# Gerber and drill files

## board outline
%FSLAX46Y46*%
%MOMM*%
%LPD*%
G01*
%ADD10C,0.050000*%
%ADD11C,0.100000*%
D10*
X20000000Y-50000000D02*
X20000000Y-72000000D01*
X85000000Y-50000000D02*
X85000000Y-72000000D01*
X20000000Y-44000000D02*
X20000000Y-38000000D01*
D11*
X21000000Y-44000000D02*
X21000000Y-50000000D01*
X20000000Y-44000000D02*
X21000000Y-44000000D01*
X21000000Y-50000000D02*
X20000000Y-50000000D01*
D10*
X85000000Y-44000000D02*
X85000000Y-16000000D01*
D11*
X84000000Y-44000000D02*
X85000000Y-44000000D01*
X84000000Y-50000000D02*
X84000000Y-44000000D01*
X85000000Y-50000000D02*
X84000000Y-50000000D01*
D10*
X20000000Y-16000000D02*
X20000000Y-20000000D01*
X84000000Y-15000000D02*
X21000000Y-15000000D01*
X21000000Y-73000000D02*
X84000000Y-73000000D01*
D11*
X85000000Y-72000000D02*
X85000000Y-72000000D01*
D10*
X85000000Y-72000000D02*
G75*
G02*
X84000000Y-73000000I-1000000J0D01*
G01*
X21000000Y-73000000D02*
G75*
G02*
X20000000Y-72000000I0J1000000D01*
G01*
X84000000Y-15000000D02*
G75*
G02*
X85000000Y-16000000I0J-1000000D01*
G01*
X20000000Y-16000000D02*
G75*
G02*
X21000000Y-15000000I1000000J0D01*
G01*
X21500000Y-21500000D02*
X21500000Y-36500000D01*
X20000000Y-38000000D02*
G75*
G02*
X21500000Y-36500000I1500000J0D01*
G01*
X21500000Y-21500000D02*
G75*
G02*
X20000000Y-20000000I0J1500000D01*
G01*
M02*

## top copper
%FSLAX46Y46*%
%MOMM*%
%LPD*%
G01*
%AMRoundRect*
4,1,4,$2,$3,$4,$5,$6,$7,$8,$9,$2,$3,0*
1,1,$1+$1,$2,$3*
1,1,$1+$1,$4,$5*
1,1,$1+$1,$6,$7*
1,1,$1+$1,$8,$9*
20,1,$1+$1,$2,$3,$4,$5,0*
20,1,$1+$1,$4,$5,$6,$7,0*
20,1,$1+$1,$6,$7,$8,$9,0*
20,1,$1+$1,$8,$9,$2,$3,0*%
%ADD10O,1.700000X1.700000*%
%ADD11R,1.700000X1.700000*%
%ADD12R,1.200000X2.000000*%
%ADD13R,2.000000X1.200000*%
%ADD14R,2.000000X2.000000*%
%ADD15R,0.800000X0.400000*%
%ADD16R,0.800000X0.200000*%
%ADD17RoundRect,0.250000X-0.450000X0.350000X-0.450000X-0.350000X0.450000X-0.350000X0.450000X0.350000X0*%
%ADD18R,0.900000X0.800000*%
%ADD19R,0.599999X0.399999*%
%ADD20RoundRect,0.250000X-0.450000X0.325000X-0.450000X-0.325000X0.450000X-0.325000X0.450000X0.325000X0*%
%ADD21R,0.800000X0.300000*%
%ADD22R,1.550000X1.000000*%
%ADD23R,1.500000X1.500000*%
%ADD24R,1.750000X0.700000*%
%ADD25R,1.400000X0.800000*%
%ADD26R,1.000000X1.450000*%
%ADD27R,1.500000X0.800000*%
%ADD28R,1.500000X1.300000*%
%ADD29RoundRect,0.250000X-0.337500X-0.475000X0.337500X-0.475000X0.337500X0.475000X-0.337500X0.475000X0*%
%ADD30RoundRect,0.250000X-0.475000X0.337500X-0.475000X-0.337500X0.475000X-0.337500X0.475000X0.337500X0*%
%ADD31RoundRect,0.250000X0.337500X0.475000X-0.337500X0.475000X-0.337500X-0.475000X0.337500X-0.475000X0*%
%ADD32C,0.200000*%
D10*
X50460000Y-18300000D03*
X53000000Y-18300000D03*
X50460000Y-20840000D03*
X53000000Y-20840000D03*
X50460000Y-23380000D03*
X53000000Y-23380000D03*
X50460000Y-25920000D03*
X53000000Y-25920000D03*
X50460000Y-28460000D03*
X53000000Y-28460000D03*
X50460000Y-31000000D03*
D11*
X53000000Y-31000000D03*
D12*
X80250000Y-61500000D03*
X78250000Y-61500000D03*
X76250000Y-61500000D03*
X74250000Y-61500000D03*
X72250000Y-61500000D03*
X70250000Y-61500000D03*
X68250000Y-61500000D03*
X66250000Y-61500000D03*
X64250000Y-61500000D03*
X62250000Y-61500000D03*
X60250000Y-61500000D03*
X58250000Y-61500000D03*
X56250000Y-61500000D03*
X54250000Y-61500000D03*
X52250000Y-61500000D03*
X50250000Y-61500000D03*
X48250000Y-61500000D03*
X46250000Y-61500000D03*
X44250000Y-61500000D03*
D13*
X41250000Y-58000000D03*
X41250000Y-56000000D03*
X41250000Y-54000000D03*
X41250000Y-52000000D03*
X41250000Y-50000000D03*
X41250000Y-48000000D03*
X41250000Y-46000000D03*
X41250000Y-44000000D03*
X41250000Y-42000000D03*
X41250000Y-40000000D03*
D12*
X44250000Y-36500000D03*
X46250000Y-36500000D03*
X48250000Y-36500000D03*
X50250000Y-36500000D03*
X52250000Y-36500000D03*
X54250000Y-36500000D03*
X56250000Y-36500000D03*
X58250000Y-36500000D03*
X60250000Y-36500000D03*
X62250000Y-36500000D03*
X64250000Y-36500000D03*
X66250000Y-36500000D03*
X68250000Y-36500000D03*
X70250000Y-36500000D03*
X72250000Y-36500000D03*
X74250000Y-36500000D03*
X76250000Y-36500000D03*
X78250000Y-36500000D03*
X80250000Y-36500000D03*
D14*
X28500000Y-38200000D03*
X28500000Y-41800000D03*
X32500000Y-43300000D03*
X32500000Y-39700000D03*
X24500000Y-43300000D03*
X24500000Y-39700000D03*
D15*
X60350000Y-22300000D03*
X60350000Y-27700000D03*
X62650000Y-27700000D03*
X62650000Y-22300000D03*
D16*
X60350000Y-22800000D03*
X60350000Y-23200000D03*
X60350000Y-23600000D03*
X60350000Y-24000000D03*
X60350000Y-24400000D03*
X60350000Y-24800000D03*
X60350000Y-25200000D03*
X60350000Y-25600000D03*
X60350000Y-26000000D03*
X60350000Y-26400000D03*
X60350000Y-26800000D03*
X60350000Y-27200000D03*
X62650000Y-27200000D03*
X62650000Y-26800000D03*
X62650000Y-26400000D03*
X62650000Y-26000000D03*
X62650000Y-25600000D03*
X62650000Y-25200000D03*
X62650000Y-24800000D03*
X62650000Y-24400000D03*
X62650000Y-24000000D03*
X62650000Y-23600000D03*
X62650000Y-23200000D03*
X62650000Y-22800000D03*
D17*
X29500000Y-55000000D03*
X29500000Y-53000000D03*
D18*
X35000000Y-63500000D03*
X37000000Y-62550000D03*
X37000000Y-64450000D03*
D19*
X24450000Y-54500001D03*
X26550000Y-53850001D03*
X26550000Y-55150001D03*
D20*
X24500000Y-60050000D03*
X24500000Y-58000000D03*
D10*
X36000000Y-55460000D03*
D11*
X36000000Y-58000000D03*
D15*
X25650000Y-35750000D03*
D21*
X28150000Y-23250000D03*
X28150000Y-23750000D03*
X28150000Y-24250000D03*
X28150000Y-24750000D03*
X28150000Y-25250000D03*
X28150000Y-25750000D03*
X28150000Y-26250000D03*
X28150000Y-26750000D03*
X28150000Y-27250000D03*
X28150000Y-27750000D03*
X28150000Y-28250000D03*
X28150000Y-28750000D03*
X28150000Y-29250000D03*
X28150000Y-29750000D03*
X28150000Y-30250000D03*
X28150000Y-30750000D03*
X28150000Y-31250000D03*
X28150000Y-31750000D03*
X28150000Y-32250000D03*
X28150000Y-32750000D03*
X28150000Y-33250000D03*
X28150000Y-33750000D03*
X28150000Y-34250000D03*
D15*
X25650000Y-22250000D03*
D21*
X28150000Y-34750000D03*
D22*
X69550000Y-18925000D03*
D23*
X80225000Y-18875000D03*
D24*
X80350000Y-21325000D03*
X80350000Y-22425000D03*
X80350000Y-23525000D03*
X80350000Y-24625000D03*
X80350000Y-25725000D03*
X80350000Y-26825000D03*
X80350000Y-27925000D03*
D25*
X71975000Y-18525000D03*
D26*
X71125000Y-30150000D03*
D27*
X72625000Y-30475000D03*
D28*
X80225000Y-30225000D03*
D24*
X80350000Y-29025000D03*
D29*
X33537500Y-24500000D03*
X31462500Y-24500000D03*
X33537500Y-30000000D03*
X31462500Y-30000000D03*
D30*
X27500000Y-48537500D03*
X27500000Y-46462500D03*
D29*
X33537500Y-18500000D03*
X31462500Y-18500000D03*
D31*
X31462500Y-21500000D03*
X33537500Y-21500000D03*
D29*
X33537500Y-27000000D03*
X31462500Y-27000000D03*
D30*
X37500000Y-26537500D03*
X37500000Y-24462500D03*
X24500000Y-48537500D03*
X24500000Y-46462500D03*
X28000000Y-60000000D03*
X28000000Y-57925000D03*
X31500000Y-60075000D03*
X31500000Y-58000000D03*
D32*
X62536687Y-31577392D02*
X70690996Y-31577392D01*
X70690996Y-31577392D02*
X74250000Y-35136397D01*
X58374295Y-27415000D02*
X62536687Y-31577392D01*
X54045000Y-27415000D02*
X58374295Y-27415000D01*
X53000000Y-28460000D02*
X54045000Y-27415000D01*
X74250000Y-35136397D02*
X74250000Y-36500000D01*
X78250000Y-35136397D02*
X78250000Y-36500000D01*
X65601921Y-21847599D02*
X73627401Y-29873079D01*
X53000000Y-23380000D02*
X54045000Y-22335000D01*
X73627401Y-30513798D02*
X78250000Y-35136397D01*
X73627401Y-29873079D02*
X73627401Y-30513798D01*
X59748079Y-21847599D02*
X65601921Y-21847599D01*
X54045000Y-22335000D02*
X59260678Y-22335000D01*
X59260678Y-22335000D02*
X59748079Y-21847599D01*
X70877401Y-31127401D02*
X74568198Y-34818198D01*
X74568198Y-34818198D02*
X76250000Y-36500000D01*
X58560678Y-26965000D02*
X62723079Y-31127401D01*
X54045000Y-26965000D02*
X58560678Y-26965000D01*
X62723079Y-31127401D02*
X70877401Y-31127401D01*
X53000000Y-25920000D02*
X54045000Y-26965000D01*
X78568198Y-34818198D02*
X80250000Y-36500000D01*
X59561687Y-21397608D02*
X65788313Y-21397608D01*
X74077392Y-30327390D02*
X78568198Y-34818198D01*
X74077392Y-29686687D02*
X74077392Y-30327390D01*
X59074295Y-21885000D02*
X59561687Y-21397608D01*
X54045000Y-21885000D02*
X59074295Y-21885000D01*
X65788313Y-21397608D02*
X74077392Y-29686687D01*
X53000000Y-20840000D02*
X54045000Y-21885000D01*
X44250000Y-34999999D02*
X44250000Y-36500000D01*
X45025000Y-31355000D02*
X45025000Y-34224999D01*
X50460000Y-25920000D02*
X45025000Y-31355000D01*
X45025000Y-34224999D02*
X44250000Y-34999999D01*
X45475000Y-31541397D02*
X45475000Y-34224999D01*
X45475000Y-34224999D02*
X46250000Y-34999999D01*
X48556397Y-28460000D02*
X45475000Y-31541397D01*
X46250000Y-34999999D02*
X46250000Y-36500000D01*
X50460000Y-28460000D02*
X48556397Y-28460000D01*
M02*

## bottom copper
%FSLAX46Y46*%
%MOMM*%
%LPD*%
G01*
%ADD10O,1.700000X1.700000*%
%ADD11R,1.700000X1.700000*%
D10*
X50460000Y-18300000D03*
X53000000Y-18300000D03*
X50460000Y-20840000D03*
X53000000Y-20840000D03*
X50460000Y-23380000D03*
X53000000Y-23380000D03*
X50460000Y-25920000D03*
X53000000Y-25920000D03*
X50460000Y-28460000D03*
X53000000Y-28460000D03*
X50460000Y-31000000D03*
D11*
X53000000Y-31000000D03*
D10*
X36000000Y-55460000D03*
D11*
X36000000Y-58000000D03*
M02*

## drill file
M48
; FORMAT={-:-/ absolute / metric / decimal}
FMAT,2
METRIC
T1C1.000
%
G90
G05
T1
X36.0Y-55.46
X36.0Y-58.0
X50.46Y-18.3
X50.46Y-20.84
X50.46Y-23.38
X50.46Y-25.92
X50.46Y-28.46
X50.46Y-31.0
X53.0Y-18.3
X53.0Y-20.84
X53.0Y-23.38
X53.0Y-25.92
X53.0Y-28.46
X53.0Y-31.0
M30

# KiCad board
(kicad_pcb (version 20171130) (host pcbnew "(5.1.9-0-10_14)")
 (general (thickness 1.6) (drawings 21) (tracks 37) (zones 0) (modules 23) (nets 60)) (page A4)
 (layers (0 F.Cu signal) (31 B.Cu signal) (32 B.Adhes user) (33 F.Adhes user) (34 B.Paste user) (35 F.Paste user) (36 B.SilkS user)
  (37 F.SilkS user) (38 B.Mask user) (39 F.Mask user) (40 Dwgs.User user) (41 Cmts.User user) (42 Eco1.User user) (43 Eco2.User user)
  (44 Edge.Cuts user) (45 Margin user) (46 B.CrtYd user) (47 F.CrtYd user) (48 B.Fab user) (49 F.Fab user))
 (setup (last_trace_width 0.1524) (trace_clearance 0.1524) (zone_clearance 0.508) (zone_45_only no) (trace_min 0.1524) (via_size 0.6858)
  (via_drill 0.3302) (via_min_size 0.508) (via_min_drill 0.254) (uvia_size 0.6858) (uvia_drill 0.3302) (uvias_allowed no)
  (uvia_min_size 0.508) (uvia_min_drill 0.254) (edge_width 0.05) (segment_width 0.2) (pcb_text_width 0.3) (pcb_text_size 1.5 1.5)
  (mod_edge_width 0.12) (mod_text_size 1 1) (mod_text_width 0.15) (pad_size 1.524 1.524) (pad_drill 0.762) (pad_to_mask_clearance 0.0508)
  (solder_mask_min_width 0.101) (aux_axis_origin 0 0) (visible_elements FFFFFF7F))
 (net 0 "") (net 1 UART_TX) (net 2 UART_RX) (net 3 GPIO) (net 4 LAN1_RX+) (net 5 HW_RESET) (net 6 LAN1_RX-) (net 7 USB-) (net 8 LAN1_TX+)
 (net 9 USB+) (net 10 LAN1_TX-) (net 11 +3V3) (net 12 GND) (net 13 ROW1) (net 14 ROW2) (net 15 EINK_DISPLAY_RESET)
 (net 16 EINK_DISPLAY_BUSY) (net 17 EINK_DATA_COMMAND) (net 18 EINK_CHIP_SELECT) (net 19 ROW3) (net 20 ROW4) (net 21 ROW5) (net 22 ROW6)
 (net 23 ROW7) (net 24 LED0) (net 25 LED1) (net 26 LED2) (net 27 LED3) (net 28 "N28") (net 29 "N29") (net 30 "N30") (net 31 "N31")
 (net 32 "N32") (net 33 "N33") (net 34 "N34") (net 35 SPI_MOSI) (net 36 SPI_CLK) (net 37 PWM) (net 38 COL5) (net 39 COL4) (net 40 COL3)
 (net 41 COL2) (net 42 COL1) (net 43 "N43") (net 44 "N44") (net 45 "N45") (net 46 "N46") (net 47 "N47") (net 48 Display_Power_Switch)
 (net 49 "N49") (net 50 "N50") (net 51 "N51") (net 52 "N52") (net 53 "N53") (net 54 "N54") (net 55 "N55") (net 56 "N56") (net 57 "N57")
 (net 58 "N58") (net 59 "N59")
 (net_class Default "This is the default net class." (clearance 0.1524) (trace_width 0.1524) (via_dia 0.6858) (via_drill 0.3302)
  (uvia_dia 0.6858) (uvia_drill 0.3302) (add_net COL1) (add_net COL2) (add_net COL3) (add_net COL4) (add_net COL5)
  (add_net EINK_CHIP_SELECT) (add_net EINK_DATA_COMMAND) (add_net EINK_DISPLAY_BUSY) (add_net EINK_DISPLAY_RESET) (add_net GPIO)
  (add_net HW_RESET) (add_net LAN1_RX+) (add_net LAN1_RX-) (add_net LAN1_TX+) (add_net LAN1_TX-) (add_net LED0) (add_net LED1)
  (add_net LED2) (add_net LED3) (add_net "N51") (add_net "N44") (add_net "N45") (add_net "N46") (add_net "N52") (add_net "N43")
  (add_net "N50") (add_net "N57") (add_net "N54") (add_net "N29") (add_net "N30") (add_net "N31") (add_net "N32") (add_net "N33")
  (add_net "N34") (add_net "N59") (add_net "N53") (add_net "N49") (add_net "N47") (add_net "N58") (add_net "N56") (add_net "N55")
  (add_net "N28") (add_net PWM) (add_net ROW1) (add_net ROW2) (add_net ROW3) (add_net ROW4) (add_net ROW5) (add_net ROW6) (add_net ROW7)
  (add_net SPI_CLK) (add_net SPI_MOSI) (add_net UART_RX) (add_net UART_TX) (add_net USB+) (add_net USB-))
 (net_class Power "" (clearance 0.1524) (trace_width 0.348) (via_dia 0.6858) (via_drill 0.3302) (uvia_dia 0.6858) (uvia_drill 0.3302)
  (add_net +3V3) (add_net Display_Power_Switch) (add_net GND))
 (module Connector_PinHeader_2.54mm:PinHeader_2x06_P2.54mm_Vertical (layer F.Cu) (at 53 31 180)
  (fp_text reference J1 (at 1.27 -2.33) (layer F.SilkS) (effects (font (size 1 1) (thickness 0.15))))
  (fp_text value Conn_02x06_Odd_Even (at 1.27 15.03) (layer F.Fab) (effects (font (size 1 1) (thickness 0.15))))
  (pad 12 thru_hole oval (at 2.54 12.7 180) (size 1.7 1.7) (drill 1) (layers *.Cu *.Mask) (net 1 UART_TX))
  (pad 11 thru_hole oval (at 0 12.7 180) (size 1.7 1.7) (drill 1) (layers *.Cu *.Mask) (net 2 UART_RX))
  (pad 10 thru_hole oval (at 2.54 10.16 180) (size 1.7 1.7) (drill 1) (layers *.Cu *.Mask) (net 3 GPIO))
  (pad 9 thru_hole oval (at 0 10.16 180) (size 1.7 1.7) (drill 1) (layers *.Cu *.Mask) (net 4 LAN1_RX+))
  (pad 8 thru_hole oval (at 2.54 7.62 180) (size 1.7 1.7) (drill 1) (layers *.Cu *.Mask) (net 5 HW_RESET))
  (pad 7 thru_hole oval (at 0 7.62 180) (size 1.7 1.7) (drill 1) (layers *.Cu *.Mask) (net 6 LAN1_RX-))
  (pad 6 thru_hole oval (at 2.54 5.08 180) (size 1.7 1.7) (drill 1) (layers *.Cu *.Mask) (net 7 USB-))
  (pad 5 thru_hole oval (at 0 5.08 180) (size 1.7 1.7) (drill 1) (layers *.Cu *.Mask) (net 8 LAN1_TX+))
  (pad 4 thru_hole oval (at 2.54 2.54 180) (size 1.7 1.7) (drill 1) (layers *.Cu *.Mask) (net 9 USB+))
  (pad 3 thru_hole oval (at 0 2.54 180) (size 1.7 1.7) (drill 1) (layers *.Cu *.Mask) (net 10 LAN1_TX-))
  (pad 2 thru_hole oval (at 2.54 0 180) (size 1.7 1.7) (drill 1) (layers *.Cu *.Mask) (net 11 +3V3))
  (pad 1 thru_hole rect (at 0 0 180) (size 1.7 1.7) (drill 1) (layers *.Cu *.Mask) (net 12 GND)))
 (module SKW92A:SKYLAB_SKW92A (layer F.Cu) (at 61.5 49)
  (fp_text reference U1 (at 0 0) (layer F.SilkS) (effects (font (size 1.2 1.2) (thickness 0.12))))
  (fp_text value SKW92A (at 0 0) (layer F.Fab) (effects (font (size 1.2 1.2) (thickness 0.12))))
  (pad 48 smd rect (at 18.75 12.5) (size 1.2 2) (layers F.Cu F.Paste F.Mask) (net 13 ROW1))
  (pad 47 smd rect (at 16.75 12.5) (size 1.2 2) (layers F.Cu F.Paste F.Mask) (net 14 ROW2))
  (pad 46 smd rect (at 14.75 12.5) (size 1.2 2) (layers F.Cu F.Paste F.Mask) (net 3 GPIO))
  (pad 45 smd rect (at 12.75 12.5) (size 1.2 2) (layers F.Cu F.Paste F.Mask) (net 5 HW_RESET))
  (pad 44 smd rect (at 10.75 12.5) (size 1.2 2) (layers F.Cu F.Paste F.Mask) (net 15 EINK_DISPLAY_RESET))
  (pad 43 smd rect (at 8.75 12.5) (size 1.2 2) (layers F.Cu F.Paste F.Mask) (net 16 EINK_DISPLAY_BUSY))
  (pad 42 smd rect (at 6.75 12.5) (size 1.2 2) (layers F.Cu F.Paste F.Mask) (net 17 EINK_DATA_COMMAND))
  (pad 41 smd rect (at 4.75 12.5) (size 1.2 2) (layers F.Cu F.Paste F.Mask) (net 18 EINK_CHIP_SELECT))
  (pad 40 smd rect (at 2.75 12.5) (size 1.2 2) (layers F.Cu F.Paste F.Mask) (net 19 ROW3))
  (pad 39 smd rect (at 0.75 12.5) (size 1.2 2) (layers F.Cu F.Paste F.Mask) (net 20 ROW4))
  (pad 38 smd rect (at -1.25 12.5) (size 1.2 2) (layers F.Cu F.Paste F.Mask) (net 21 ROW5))
  (pad 37 smd rect (at -3.25 12.5) (size 1.2 2) (layers F.Cu F.Paste F.Mask) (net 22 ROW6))
  (pad 36 smd rect (at -5.25 12.5) (size 1.2 2) (layers F.Cu F.Paste F.Mask) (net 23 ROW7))
  (pad 35 smd rect (at -7.25 12.5) (size 1.2 2) (layers F.Cu F.Paste F.Mask) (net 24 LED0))
  (pad 34 smd rect (at -9.25 12.5) (size 1.2 2) (layers F.Cu F.Paste F.Mask) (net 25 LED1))
  (pad 33 smd rect (at -11.25 12.5) (size 1.2 2) (layers F.Cu F.Paste F.Mask) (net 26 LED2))
  (pad 32 smd rect (at -13.25 12.5) (size 1.2 2) (layers F.Cu F.Paste F.Mask) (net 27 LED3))
  (pad 31 smd rect (at -15.25 12.5) (size 1.2 2) (layers F.Cu F.Paste F.Mask) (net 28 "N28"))
  (pad 30 smd rect (at -17.25 12.5) (size 1.2 2) (layers F.Cu F.Paste F.Mask) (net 12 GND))
  (pad 29 smd rect (at -20.25 9 90) (size 1.2 2) (layers F.Cu F.Paste F.Mask) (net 11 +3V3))
  (pad 28 smd rect (at -20.25 7 90) (size 1.2 2) (layers F.Cu F.Paste F.Mask) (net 11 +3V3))
  (pad 27 smd rect (at -20.25 5 90) (size 1.2 2) (layers F.Cu F.Paste F.Mask) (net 12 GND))
  (pad 26 smd rect (at -20.25 3 90) (size 1.2 2) (layers F.Cu F.Paste F.Mask) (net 1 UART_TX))
  (pad 25 smd rect (at -20.25 1 90) (size 1.2 2) (layers F.Cu F.Paste F.Mask) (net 2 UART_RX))
  (pad 24 smd rect (at -20.25 -1 90) (size 1.2 2) (layers F.Cu F.Paste F.Mask) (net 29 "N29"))
  (pad 23 smd rect (at -20.25 -3 90) (size 1.2 2) (layers F.Cu F.Paste F.Mask) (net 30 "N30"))
  (pad 22 smd rect (at -20.25 -5 90) (size 1.2 2) (layers F.Cu F.Paste F.Mask) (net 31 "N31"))
  (pad 21 smd rect (at -20.25 -7 90) (size 1.2 2) (layers F.Cu F.Paste F.Mask) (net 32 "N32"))
  (pad 20 smd rect (at -20.25 -9 90) (size 1.2 2) (layers F.Cu F.Paste F.Mask) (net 12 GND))
  (pad 19 smd rect (at -17.25 -12.5) (size 1.2 2) (layers F.Cu F.Paste F.Mask) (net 7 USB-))
  (pad 18 smd rect (at -15.25 -12.5) (size 1.2 2) (layers F.Cu F.Paste F.Mask) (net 9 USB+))
  (pad 17 smd rect (at -13.25 -12.5) (size 1.2 2) (layers F.Cu F.Paste F.Mask) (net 12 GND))
  (pad 16 smd rect (at -11.25 -12.5) (size 1.2 2) (layers F.Cu F.Paste F.Mask) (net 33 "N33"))
  (pad 15 smd rect (at -9.25 -12.5) (size 1.2 2) (layers F.Cu F.Paste F.Mask) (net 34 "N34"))
  (pad 14 smd rect (at -7.25 -12.5) (size 1.2 2) (layers F.Cu F.Paste F.Mask) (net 12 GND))
  (pad 13 smd rect (at -5.25 -12.5) (size 1.2 2) (layers F.Cu F.Paste F.Mask) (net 12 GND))
  (pad 12 smd rect (at -3.25 -12.5) (size 1.2 2) (layers F.Cu F.Paste F.Mask) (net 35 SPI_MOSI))
  (pad 11 smd rect (at -1.25 -12.5) (size 1.2 2) (layers F.Cu F.Paste F.Mask) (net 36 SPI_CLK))
  (pad 10 smd rect (at 0.75 -12.5) (size 1.2 2) (layers F.Cu F.Paste F.Mask) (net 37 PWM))
  (pad 9 smd rect (at 2.75 -12.5) (size 1.2 2) (layers F.Cu F.Paste F.Mask) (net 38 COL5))
  (pad 8 smd rect (at 4.75 -12.5) (size 1.2 2) (layers F.Cu F.Paste F.Mask) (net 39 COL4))
  (pad 7 smd rect (at 6.75 -12.5) (size 1.2 2) (layers F.Cu F.Paste F.Mask) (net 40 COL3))
  (pad 6 smd rect (at 8.75 -12.5) (size 1.2 2) (layers F.Cu F.Paste F.Mask) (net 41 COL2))
  (pad 5 smd rect (at 10.75 -12.5) (size 1.2 2) (layers F.Cu F.Paste F.Mask) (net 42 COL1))
  (pad 4 smd rect (at 12.75 -12.5) (size 1.2 2) (layers F.Cu F.Paste F.Mask) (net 10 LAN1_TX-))
  (pad 3 smd rect (at 14.75 -12.5) (size 1.2 2) (layers F.Cu F.Paste F.Mask) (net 8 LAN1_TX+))
  (pad 2 smd rect (at 16.75 -12.5) (size 1.2 2) (layers F.Cu F.Paste F.Mask) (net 6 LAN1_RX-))
  (pad 1 smd rect (at 18.75 -12.5) (size 1.2 2) (layers F.Cu F.Paste F.Mask) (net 4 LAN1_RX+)))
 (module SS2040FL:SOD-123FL (layer F.Cu) (at 28.5 40 90)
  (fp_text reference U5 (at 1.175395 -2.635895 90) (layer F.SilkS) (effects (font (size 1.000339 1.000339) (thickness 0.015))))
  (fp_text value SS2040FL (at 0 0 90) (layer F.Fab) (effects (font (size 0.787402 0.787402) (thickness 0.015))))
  (pad 2 smd rect (at 1.8 0 90) (size 2 2) (layers F.Cu F.Paste F.Mask) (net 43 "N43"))
  (pad 1 smd rect (at -1.8 0 90) (size 2 2) (layers F.Cu F.Paste F.Mask) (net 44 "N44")))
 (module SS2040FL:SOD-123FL (layer F.Cu) (at 32.5 41.5 270)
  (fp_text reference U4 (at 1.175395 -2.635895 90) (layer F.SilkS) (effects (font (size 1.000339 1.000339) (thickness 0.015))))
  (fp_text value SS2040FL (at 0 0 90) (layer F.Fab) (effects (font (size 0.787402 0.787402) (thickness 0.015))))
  (pad 2 smd rect (at 1.8 0 270) (size 2 2) (layers F.Cu F.Paste F.Mask) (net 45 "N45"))
  (pad 1 smd rect (at -1.8 0 270) (size 2 2) (layers F.Cu F.Paste F.Mask) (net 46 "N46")))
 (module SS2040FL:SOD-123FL (layer F.Cu) (at 24.5 41.5 270)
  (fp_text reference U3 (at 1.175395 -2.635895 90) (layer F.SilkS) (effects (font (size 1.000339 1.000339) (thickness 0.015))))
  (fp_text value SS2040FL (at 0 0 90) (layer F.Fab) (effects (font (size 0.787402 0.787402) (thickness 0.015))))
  (pad 2 smd rect (at 1.8 0 270) (size 2 2) (layers F.Cu F.Paste F.Mask) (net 44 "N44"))
  (pad 1 smd rect (at -1.8 0 270) (size 2 2) (layers F.Cu F.Paste F.Mask) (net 12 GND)))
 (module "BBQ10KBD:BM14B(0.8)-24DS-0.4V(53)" (layer F.Cu) (at 61.5 25 270)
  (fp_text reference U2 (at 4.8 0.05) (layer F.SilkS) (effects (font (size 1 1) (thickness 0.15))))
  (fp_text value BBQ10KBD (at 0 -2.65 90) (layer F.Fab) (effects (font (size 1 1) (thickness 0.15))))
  (pad 28 smd rect (at -2.7 1.15 270) (size 0.4 0.8) (layers F.Cu F.Paste F.Mask) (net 12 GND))
  (pad 15 smd rect (at 2.7 1.15 270) (size 0.4 0.8) (layers F.Cu F.Paste F.Mask) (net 12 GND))
  (pad 14 smd rect (at 2.7 -1.15 270) (size 0.4 0.8) (layers F.Cu F.Paste F.Mask) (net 12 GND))
  (pad 1 smd rect (at -2.7 -1.15 270) (size 0.4 0.8) (layers F.Cu F.Paste F.Mask) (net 12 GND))
  (pad 27 smd rect (at -2.2 1.15 270) (size 0.2 0.8) (layers F.Cu F.Paste F.Mask) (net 23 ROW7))
  (pad 26 smd rect (at -1.8 1.15 270) (size 0.2 0.8) (layers F.Cu F.Paste F.Mask) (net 24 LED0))
  (pad 25 smd rect (at -1.4 1.15 270) (size 0.2 0.8) (layers F.Cu F.Paste F.Mask) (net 26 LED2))
  (pad 24 smd rect (at -1 1.15 270) (size 0.2 0.8) (layers F.Cu F.Paste F.Mask) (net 25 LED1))
  (pad 23 smd rect (at -0.6 1.15 270) (size 0.2 0.8) (layers F.Cu F.Paste F.Mask) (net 27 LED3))
  (pad 22 smd rect (at -0.2 1.15 270) (size 0.2 0.8) (layers F.Cu F.Paste F.Mask) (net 22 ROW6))
  (pad 21 smd rect (at 0.2 1.15 270) (size 0.2 0.8) (layers F.Cu F.Paste F.Mask) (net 21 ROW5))
  (pad 20 smd rect (at 0.6 1.15 270) (size 0.2 0.8) (layers F.Cu F.Paste F.Mask) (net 20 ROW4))
  (pad 19 smd rect (at 1 1.15 270) (size 0.2 0.8) (layers F.Cu F.Paste F.Mask) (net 38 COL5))
  (pad 18 smd rect (at 1.4 1.15 270) (size 0.2 0.8) (layers F.Cu F.Paste F.Mask) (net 19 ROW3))
  (pad 17 smd rect (at 1.8 1.15 270) (size 0.2 0.8) (layers F.Cu F.Paste F.Mask) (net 39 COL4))
  (pad 16 smd rect (at 2.2 1.15 270) (size 0.2 0.8) (layers F.Cu F.Paste F.Mask) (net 12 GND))
  (pad 13 smd rect (at 2.2 -1.15 270) (size 0.2 0.8) (layers F.Cu F.Paste F.Mask) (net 12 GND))
  (pad 12 smd rect (at 1.8 -1.15 270) (size 0.2 0.8) (layers F.Cu F.Paste F.Mask) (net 12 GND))
  (pad 11 smd rect (at 1.4 -1.15 270) (size 0.2 0.8) (layers F.Cu F.Paste F.Mask) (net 12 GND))
  (pad 10 smd rect (at 1 -1.15 270) (size 0.2 0.8) (layers F.Cu F.Paste F.Mask) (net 40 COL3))
  (pad 9 smd rect (at 0.6 -1.15 270) (size 0.2 0.8) (layers F.Cu F.Paste F.Mask) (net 41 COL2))
  (pad 8 smd rect (at 0.2 -1.15 270) (size 0.2 0.8) (layers F.Cu F.Paste F.Mask) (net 14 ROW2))
  (pad 7 smd rect (at -0.2 -1.15 270) (size 0.2 0.8) (layers F.Cu F.Paste F.Mask) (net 42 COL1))
  (pad 6 smd rect (at -0.6 -1.15 270) (size 0.2 0.8) (layers F.Cu F.Paste F.Mask) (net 13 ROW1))
  (pad 5 smd rect (at -1 -1.15 270) (size 0.2 0.8) (layers F.Cu F.Paste F.Mask) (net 12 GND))
  (pad 4 smd rect (at -1.4 -1.15 270) (size 0.2 0.8) (layers F.Cu F.Paste F.Mask) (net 12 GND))
  (pad 3 smd rect (at -1.8 -1.15 270) (size 0.2 0.8) (layers F.Cu F.Paste F.Mask) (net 37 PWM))
  (pad 2 smd rect (at -2.2 -1.15 270) (size 0.2 0.8) (layers F.Cu F.Paste F.Mask) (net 11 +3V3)))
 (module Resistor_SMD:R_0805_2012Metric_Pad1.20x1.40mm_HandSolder (layer F.Cu) (at 29.5 54 270)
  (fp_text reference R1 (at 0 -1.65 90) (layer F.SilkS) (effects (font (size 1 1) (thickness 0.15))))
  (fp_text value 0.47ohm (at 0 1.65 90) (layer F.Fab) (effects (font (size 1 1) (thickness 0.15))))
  (pad 2 smd roundrect (at 1 0 270) (size 1.2 1.4) (layers F.Cu F.Paste F.Mask) (roundrect_rratio 0.208333) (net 12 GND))
  (pad 1 smd roundrect (at -1 0 270) (size 1.2 1.4) (layers F.Cu F.Paste F.Mask) (roundrect_rratio 0.208333) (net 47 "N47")))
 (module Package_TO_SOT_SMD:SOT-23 (layer F.Cu) (at 36 63.5 180)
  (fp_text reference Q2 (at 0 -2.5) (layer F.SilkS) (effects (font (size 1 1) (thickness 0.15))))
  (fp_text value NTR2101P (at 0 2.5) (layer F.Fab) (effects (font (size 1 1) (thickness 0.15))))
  (pad 3 smd rect (at 1 0 180) (size 0.9 0.8) (layers F.Cu F.Paste F.Mask) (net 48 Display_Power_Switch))
  (pad 2 smd rect (at -1 0.95 180) (size 0.9 0.8) (layers F.Cu F.Paste F.Mask) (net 11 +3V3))
  (pad 1 smd rect (at -1 -0.95 180) (size 0.9 0.8) (layers F.Cu F.Paste F.Mask) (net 28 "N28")))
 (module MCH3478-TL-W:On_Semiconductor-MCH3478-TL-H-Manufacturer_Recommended (layer F.Cu) (at 25.5 54.5 180)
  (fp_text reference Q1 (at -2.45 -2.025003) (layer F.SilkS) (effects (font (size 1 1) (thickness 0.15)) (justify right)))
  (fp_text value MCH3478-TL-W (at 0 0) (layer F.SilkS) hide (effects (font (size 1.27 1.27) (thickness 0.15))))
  (pad 3 smd rect (at 1.05 -0.000001 270) (size 0.399999 0.599999) (layers F.Cu F.Paste F.Mask) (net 45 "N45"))
  (pad 2 smd rect (at -1.05 0.649999 270) (size 0.399999 0.599999) (layers F.Cu F.Paste F.Mask) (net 47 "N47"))
  (pad 1 smd rect (at -1.05 -0.650001 270) (size 0.399999 0.599999) (layers F.Cu F.Paste F.Mask) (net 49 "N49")))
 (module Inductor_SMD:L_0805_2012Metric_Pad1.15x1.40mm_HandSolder (layer F.Cu) (at 24.5 59.025 270)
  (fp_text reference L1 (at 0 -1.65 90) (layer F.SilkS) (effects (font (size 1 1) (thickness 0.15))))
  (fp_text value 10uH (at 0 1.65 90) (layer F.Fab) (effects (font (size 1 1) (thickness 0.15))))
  (pad 2 smd roundrect (at 1.025 0 270) (size 1.15 1.4) (layers F.Cu F.Paste F.Mask) (roundrect_rratio 0.217391)
   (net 48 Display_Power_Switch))
  (pad 1 smd roundrect (at -1.025 0 270) (size 1.15 1.4) (layers F.Cu F.Paste F.Mask) (roundrect_rratio 0.217391) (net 45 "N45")))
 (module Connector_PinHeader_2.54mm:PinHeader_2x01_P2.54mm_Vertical (layer F.Cu) (at 36 58 90)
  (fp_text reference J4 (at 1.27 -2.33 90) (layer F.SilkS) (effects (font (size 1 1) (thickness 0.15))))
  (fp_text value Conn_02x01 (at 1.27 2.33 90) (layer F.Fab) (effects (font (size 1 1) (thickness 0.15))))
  (pad 2 thru_hole oval (at 2.54 0 90) (size 1.7 1.7) (drill 1) (layers *.Cu *.Mask) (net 12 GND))
  (pad 1 thru_hole rect (at 0 0 90) (size 1.7 1.7) (drill 1) (layers *.Cu *.Mask) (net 11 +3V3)))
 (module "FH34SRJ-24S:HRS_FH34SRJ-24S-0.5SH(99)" (layer F.Cu) (at 27 29 270)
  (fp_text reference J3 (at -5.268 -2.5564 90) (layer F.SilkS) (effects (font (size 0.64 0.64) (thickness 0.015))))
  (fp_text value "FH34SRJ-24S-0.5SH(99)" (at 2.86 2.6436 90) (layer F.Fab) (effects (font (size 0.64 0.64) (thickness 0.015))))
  (pad S2 smd rect (at 6.75 1.35 270) (size 0.4 0.8) (layers F.Cu F.Paste F.Mask) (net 12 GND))
  (pad 24 smd rect (at -5.75 -1.15 270) (size 0.3 0.8) (layers F.Cu F.Mask) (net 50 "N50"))
  (pad 23 smd rect (at -5.25 -1.15 270) (size 0.3 0.8) (layers F.Cu F.Mask) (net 43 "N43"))
  (pad 22 smd rect (at -4.75 -1.15 270) (size 0.3 0.8) (layers F.Cu F.Mask) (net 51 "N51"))
  (pad 21 smd rect (at -4.25 -1.15 270) (size 0.3 0.8) (layers F.Cu F.Mask) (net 46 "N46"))
  (pad 20 smd rect (at -3.75 -1.15 270) (size 0.3 0.8) (layers F.Cu F.Mask) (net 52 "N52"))
  (pad 19 smd rect (at -3.25 -1.15 270) (size 0.3 0.8) (layers F.Cu F.Mask) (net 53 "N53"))
  (pad 18 smd rect (at -2.75 -1.15 270) (size 0.3 0.8) (layers F.Cu F.Mask) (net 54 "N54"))
  (pad 17 smd rect (at -2.25 -1.15 270) (size 0.3 0.8) (layers F.Cu F.Mask) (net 12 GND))
  (pad 16 smd rect (at -1.75 -1.15 270) (size 0.3 0.8) (layers F.Cu F.Mask) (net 48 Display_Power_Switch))
  (pad 15 smd rect (at -1.25 -1.15 270) (size 0.3 0.8) (layers F.Cu F.Mask) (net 48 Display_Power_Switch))
  (pad 14 smd rect (at -0.75 -1.15 270) (size 0.3 0.8) (layers F.Cu F.Mask) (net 35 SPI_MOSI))
  (pad 13 smd rect (at -0.25 -1.15 270) (size 0.3 0.8) (layers F.Cu F.Mask) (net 36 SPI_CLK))
  (pad 12 smd rect (at 0.25 -1.15 270) (size 0.3 0.8) (layers F.Cu F.Mask) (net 18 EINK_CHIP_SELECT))
  (pad 11 smd rect (at 0.75 -1.15 270) (size 0.3 0.8) (layers F.Cu F.Mask) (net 17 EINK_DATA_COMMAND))
  (pad 10 smd rect (at 1.25 -1.15 270) (size 0.3 0.8) (layers F.Cu F.Mask) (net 15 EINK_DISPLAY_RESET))
  (pad 9 smd rect (at 1.75 -1.15 270) (size 0.3 0.8) (layers F.Cu F.Mask) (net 16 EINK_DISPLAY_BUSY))
  (pad 8 smd rect (at 2.25 -1.15 270) (size 0.3 0.8) (layers F.Cu F.Mask) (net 12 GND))
  (pad 7 smd rect (at 2.75 -1.15 270) (size 0.3 0.8) (layers F.Cu F.Mask) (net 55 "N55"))
  (pad 6 smd rect (at 3.25 -1.15 270) (size 0.3 0.8) (layers F.Cu F.Mask) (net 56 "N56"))
  (pad 5 smd rect (at 3.75 -1.15 270) (size 0.3 0.8) (layers F.Cu F.Mask) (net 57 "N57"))
  (pad 4 smd rect (at 4.25 -1.15 270) (size 0.3 0.8) (layers F.Cu F.Mask) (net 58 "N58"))
  (pad 3 smd rect (at 4.75 -1.15 270) (size 0.3 0.8) (layers F.Cu F.Mask) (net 47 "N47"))
  (pad 2 smd rect (at 5.25 -1.15 270) (size 0.3 0.8) (layers F.Cu F.Mask) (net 49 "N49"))
  (pad S1 smd rect (at -6.75 1.35 270) (size 0.4 0.8) (layers F.Cu F.Paste F.Mask) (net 12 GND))
  (pad 1 smd rect (at 5.75 -1.15 270) (size 0.3 0.8) (layers F.Cu F.Mask) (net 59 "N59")))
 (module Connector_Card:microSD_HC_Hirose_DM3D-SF (layer F.Cu) (at 75 24.5 90)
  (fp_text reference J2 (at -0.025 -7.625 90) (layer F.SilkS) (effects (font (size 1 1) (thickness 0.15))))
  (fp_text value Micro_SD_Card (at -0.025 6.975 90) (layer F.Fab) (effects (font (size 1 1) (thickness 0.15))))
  (pad 10 smd rect (at 5.575 -5.45 90) (size 1 1.55) (layers F.Cu F.Paste F.Mask))
  (pad 11 smd rect (at 5.625 5.225 90) (size 1.5 1.5) (layers F.Cu F.Paste F.Mask))
  (pad 1 smd rect (at 3.175 5.35 90) (size 0.7 1.75) (layers F.Cu F.Paste F.Mask) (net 29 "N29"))
  (pad 2 smd rect (at 2.075 5.35 90) (size 0.7 1.75) (layers F.Cu F.Paste F.Mask) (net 30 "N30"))
  (pad 3 smd rect (at 0.975 5.35 90) (size 0.7 1.75) (layers F.Cu F.Paste F.Mask) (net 31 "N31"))
  (pad 4 smd rect (at -0.125 5.35 90) (size 0.7 1.75) (layers F.Cu F.Paste F.Mask) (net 11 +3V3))
  (pad 5 smd rect (at -1.225 5.35 90) (size 0.7 1.75) (layers F.Cu F.Paste F.Mask) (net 32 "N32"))
  (pad 6 smd rect (at -2.325 5.35 90) (size 0.7 1.75) (layers F.Cu F.Paste F.Mask) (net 12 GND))
  (pad 7 smd rect (at -3.425 5.35 90) (size 0.7 1.75) (layers F.Cu F.Paste F.Mask) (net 33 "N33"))
  (pad 11 smd rect (at 5.975 -3.025 90) (size 0.8 1.4) (layers F.Cu F.Paste F.Mask))
  (pad 9 smd rect (at -5.65 -3.875 90) (size 1.45 1) (layers F.Cu F.Paste F.Mask) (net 12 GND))
  (pad 11 smd rect (at -5.975 -2.375 90) (size 0.8 1.5) (layers F.Cu F.Paste F.Mask))
  (pad 11 smd rect (at -5.725 5.225 90) (size 1.3 1.5) (layers F.Cu F.Paste F.Mask))
  (pad 8 smd rect (at -4.525 5.35 90) (size 0.7 1.75) (layers F.Cu F.Paste F.Mask) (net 34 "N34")))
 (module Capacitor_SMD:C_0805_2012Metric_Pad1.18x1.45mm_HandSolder (layer F.Cu) (at 32.5 24.5)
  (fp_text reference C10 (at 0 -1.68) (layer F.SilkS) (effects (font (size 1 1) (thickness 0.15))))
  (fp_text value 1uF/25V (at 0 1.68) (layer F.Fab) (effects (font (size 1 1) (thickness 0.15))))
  (pad 2 smd roundrect (at 1.0375 0) (size 1.175 1.45) (layers F.Cu F.Paste F.Mask) (roundrect_rratio 0.212766) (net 12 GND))
  (pad 1 smd roundrect (at -1.0375 0) (size 1.175 1.45) (layers F.Cu F.Paste F.Mask) (roundrect_rratio 0.212766) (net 51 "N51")))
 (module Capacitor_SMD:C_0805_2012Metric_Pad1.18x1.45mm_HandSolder (layer F.Cu) (at 32.5 30)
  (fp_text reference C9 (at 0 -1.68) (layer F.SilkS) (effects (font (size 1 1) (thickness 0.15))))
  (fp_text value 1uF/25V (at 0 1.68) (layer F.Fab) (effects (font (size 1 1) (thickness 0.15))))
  (pad 2 smd roundrect (at 1.0375 0) (size 1.175 1.45) (layers F.Cu F.Paste F.Mask) (roundrect_rratio 0.212766) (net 12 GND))
  (pad 1 smd roundrect (at -1.0375 0) (size 1.175 1.45) (layers F.Cu F.Paste F.Mask) (roundrect_rratio 0.212766) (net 54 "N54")))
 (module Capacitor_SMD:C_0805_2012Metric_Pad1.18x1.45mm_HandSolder (layer F.Cu) (at 27.5 47.5 270)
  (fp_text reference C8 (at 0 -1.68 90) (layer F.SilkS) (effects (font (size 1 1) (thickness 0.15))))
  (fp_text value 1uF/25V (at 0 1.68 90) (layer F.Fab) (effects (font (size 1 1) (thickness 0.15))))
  (pad 2 smd roundrect (at 1.0375 0 270) (size 1.175 1.45) (layers F.Cu F.Paste F.Mask) (roundrect_rratio 0.212766) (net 12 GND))
  (pad 1 smd roundrect (at -1.0375 0 270) (size 1.175 1.45) (layers F.Cu F.Paste F.Mask) (roundrect_rratio 0.212766) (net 57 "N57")))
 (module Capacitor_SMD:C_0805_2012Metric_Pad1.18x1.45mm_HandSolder (layer F.Cu) (at 32.5 18.5)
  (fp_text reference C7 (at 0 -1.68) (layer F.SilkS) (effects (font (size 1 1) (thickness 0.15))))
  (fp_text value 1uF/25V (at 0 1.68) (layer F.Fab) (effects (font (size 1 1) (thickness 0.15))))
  (pad 2 smd roundrect (at 1.0375 0) (size 1.175 1.45) (layers F.Cu F.Paste F.Mask) (roundrect_rratio 0.212766) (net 12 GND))
  (pad 1 smd roundrect (at -1.0375 0) (size 1.175 1.45) (layers F.Cu F.Paste F.Mask) (roundrect_rratio 0.212766) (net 50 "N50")))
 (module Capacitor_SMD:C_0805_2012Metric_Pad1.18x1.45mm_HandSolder (layer F.Cu) (at 32.5 21.5 180)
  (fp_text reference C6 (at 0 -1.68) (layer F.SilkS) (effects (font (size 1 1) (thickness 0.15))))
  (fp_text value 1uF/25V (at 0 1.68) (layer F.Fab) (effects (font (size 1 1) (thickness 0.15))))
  (pad 2 smd roundrect (at 1.0375 0 180) (size 1.175 1.45) (layers F.Cu F.Paste F.Mask) (roundrect_rratio 0.212766) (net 43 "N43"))
  (pad 1 smd roundrect (at -1.0375 0 180) (size 1.175 1.45) (layers F.Cu F.Paste F.Mask) (roundrect_rratio 0.212766) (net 12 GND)))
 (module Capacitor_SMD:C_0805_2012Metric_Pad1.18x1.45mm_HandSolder (layer F.Cu) (at 32.5 27)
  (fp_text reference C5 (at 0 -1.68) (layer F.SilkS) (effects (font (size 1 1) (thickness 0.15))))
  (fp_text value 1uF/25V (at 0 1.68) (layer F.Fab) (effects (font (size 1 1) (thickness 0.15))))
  (pad 2 smd roundrect (at 1.0375 0) (size 1.175 1.45) (layers F.Cu F.Paste F.Mask) (roundrect_rratio 0.212766) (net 12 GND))
  (pad 1 smd roundrect (at -1.0375 0) (size 1.175 1.45) (layers F.Cu F.Paste F.Mask) (roundrect_rratio 0.212766) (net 52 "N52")))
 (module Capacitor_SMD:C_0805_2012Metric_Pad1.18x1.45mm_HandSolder (layer F.Cu) (at 37.5 25.5 270)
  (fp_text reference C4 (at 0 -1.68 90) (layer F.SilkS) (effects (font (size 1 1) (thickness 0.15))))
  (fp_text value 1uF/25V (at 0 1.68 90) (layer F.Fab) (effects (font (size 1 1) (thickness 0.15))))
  (pad 2 smd roundrect (at 1.0375 0 270) (size 1.175 1.45) (layers F.Cu F.Paste F.Mask) (roundrect_rratio 0.212766) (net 46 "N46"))
  (pad 1 smd roundrect (at -1.0375 0 270) (size 1.175 1.45) (layers F.Cu F.Paste F.Mask) (roundrect_rratio 0.212766) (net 12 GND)))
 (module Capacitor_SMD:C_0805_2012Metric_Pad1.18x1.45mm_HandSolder (layer F.Cu) (at 24.5 47.5 270)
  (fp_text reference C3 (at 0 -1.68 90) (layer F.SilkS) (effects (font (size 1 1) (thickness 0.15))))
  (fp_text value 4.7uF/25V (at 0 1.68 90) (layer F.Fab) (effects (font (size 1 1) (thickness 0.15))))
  (pad 2 smd roundrect (at 1.0375 0 270) (size 1.175 1.45) (layers F.Cu F.Paste F.Mask) (roundrect_rratio 0.212766) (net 45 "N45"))
  (pad 1 smd roundrect (at -1.0375 0 270) (size 1.175 1.45) (layers F.Cu F.Paste F.Mask) (roundrect_rratio 0.212766) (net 44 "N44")))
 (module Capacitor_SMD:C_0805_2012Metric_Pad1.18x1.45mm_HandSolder (layer F.Cu) (at 28 58.9625 270)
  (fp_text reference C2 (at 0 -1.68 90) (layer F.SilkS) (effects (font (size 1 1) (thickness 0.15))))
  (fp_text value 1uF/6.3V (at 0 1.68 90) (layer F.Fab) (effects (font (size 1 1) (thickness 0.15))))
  (pad 2 smd roundrect (at 1.0375 0 270) (size 1.175 1.45) (layers F.Cu F.Paste F.Mask) (roundrect_rratio 0.212766)
   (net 48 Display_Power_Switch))
  (pad 1 smd roundrect (at -1.0375 0 270) (size 1.175 1.45) (layers F.Cu F.Paste F.Mask) (roundrect_rratio 0.212766) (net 12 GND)))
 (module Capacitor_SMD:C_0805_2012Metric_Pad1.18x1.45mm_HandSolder (layer F.Cu) (at 31.5 59.0375 270)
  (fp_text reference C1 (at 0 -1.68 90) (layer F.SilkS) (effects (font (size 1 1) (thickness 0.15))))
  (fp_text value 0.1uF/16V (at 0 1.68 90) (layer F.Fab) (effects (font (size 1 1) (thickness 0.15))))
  (pad 2 smd roundrect (at 1.0375 0 270) (size 1.175 1.45) (layers F.Cu F.Paste F.Mask) (roundrect_rratio 0.212766)
   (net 48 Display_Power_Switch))
  (pad 1 smd roundrect (at -1.0375 0 270) (size 1.175 1.45) (layers F.Cu F.Paste F.Mask) (roundrect_rratio 0.212766) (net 12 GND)))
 (gr_line (start 20 50) (end 20 72) (layer Edge.Cuts) (width 0.05))
 (gr_line (start 85 50) (end 85 72) (layer Edge.Cuts) (width 0.05))
 (gr_line (start 20 44) (end 20 38) (layer Edge.Cuts) (width 0.05))
 (gr_line (start 21 44) (end 21 50) (layer Edge.Cuts) (width 0.1))
 (gr_line (start 20 44) (end 21 44) (layer Edge.Cuts) (width 0.1))
 (gr_line (start 21 50) (end 20 50) (layer Edge.Cuts) (width 0.1))
 (gr_line (start 85 44) (end 85 16) (layer Edge.Cuts) (width 0.05))
 (gr_line (start 84 44) (end 85 44) (layer Edge.Cuts) (width 0.1))
 (gr_line (start 84 50) (end 84 44) (layer Edge.Cuts) (width 0.1))
 (gr_line (start 85 50) (end 84 50) (layer Edge.Cuts) (width 0.1))
 (gr_line (start 20 16) (end 20 20) (layer Edge.Cuts) (width 0.05))
 (gr_line (start 84 15) (end 21 15) (layer Edge.Cuts) (width 0.05))
 (gr_line (start 21 73) (end 84 73) (layer Edge.Cuts) (width 0.05))
 (gr_line (start 85 72) (end 85 72) (layer Edge.Cuts) (width 0.1))
 (gr_arc (start 84 72) (end 84 73) (angle -90) (layer Edge.Cuts) (width 0.05))
 (gr_arc (start 21 72) (end 20 72) (angle -90) (layer Edge.Cuts) (width 0.05))
 (gr_arc (start 84 16) (end 85 16) (angle -90) (layer Edge.Cuts) (width 0.05))
 (gr_arc (start 21 16) (end 21 15) (angle -90) (layer Edge.Cuts) (width 0.05))
 (gr_line (start 21.5 21.5) (end 21.5 36.5) (layer Edge.Cuts) (width 0.05))
 (gr_arc (start 21.5 38) (end 21.5 36.5) (angle -90) (layer Edge.Cuts) (width 0.05))
 (gr_arc (start 21.5 20) (end 20 20) (angle -90) (layer Edge.Cuts) (width 0.05))
 (segment (start 62.536687 31.577392) (end 70.690996 31.577392) (width 0.2) (layer F.Cu) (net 10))
 (segment (start 70.690996 31.577392) (end 74.25 35.136397) (width 0.2) (layer F.Cu) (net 10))
 (segment (start 58.374295 27.415) (end 62.536687 31.577392) (width 0.2) (layer F.Cu) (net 10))
 (segment (start 54.045 27.415) (end 58.374295 27.415) (width 0.2) (layer F.Cu) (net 10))
 (segment (start 53 28.46) (end 54.045 27.415) (width 0.2) (layer F.Cu) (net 10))
 (segment (start 74.25 35.136397) (end 74.25 36.5) (width 0.2) (layer F.Cu) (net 10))
 (segment (start 78.25 35.136397) (end 78.25 36.5) (width 0.2) (layer F.Cu) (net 6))
 (segment (start 65.601921 21.847599) (end 73.627401 29.873079) (width 0.2) (layer F.Cu) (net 6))
 (segment (start 53 23.38) (end 54.045 22.335) (width 0.2) (layer F.Cu) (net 6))
 (segment (start 73.627401 30.513798) (end 78.25 35.136397) (width 0.2) (layer F.Cu) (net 6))
 (segment (start 73.627401 29.873079) (end 73.627401 30.513798) (width 0.2) (layer F.Cu) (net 6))
 (segment (start 59.748079 21.847599) (end 65.601921 21.847599) (width 0.2) (layer F.Cu) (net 6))
 (segment (start 54.045 22.335) (end 59.260678 22.335) (width 0.2) (layer F.Cu) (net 6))
 (segment (start 59.260678 22.335) (end 59.748079 21.847599) (width 0.2) (layer F.Cu) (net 6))
 (segment (start 70.877401 31.127401) (end 74.568198 34.818198) (width 0.2) (layer F.Cu) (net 8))
 (segment (start 74.568198 34.818198) (end 76.25 36.5) (width 0.2) (layer F.Cu) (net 8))
 (segment (start 58.560678 26.965) (end 62.723079 31.127401) (width 0.2) (layer F.Cu) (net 8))
 (segment (start 54.045 26.965) (end 58.560678 26.965) (width 0.2) (layer F.Cu) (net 8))
 (segment (start 62.723079 31.127401) (end 70.877401 31.127401) (width 0.2) (layer F.Cu) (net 8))
 (segment (start 53 25.92) (end 54.045 26.965) (width 0.2) (layer F.Cu) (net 8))
 (segment (start 78.568198 34.818198) (end 80.25 36.5) (width 0.2) (layer F.Cu) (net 4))
 (segment (start 59.561687 21.397608) (end 65.788313 21.397608) (width 0.2) (layer F.Cu) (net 4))
 (segment (start 74.077392 30.32739) (end 78.568198 34.818198) (width 0.2) (layer F.Cu) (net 4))
 (segment (start 74.077392 29.686687) (end 74.077392 30.32739) (width 0.2) (layer F.Cu) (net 4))
 (segment (start 59.074295 21.885) (end 59.561687 21.397608) (width 0.2) (layer F.Cu) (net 4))
 (segment (start 54.045 21.885) (end 59.074295 21.885) (width 0.2) (layer F.Cu) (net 4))
 (segment (start 65.788313 21.397608) (end 74.077392 29.686687) (width 0.2) (layer F.Cu) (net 4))
 (segment (start 53 20.84) (end 54.045 21.885) (width 0.2) (layer F.Cu) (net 4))
 (segment (start 44.25 34.999999) (end 44.25 36.5) (width 0.2) (layer F.Cu) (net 7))
 (segment (start 45.025 31.355) (end 45.025 34.224999) (width 0.2) (layer F.Cu) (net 7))
 (segment (start 50.46 25.92) (end 45.025 31.355) (width 0.2) (layer F.Cu) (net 7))
 (segment (start 45.025 34.224999) (end 44.25 34.999999) (width 0.2) (layer F.Cu) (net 7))
 (segment (start 45.475 31.541397) (end 45.475 34.224999) (width 0.2) (layer F.Cu) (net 9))
 (segment (start 45.475 34.224999) (end 46.25 34.999999) (width 0.2) (layer F.Cu) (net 9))
 (segment (start 48.556397 28.46) (end 45.475 31.541397) (width 0.2) (layer F.Cu) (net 9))
 (segment (start 46.25 34.999999) (end 46.25 36.5) (width 0.2) (layer F.Cu) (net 9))
 (segment (start 50.46 28.46) (end 48.556397 28.46) (width 0.2) (layer F.Cu) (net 9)))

